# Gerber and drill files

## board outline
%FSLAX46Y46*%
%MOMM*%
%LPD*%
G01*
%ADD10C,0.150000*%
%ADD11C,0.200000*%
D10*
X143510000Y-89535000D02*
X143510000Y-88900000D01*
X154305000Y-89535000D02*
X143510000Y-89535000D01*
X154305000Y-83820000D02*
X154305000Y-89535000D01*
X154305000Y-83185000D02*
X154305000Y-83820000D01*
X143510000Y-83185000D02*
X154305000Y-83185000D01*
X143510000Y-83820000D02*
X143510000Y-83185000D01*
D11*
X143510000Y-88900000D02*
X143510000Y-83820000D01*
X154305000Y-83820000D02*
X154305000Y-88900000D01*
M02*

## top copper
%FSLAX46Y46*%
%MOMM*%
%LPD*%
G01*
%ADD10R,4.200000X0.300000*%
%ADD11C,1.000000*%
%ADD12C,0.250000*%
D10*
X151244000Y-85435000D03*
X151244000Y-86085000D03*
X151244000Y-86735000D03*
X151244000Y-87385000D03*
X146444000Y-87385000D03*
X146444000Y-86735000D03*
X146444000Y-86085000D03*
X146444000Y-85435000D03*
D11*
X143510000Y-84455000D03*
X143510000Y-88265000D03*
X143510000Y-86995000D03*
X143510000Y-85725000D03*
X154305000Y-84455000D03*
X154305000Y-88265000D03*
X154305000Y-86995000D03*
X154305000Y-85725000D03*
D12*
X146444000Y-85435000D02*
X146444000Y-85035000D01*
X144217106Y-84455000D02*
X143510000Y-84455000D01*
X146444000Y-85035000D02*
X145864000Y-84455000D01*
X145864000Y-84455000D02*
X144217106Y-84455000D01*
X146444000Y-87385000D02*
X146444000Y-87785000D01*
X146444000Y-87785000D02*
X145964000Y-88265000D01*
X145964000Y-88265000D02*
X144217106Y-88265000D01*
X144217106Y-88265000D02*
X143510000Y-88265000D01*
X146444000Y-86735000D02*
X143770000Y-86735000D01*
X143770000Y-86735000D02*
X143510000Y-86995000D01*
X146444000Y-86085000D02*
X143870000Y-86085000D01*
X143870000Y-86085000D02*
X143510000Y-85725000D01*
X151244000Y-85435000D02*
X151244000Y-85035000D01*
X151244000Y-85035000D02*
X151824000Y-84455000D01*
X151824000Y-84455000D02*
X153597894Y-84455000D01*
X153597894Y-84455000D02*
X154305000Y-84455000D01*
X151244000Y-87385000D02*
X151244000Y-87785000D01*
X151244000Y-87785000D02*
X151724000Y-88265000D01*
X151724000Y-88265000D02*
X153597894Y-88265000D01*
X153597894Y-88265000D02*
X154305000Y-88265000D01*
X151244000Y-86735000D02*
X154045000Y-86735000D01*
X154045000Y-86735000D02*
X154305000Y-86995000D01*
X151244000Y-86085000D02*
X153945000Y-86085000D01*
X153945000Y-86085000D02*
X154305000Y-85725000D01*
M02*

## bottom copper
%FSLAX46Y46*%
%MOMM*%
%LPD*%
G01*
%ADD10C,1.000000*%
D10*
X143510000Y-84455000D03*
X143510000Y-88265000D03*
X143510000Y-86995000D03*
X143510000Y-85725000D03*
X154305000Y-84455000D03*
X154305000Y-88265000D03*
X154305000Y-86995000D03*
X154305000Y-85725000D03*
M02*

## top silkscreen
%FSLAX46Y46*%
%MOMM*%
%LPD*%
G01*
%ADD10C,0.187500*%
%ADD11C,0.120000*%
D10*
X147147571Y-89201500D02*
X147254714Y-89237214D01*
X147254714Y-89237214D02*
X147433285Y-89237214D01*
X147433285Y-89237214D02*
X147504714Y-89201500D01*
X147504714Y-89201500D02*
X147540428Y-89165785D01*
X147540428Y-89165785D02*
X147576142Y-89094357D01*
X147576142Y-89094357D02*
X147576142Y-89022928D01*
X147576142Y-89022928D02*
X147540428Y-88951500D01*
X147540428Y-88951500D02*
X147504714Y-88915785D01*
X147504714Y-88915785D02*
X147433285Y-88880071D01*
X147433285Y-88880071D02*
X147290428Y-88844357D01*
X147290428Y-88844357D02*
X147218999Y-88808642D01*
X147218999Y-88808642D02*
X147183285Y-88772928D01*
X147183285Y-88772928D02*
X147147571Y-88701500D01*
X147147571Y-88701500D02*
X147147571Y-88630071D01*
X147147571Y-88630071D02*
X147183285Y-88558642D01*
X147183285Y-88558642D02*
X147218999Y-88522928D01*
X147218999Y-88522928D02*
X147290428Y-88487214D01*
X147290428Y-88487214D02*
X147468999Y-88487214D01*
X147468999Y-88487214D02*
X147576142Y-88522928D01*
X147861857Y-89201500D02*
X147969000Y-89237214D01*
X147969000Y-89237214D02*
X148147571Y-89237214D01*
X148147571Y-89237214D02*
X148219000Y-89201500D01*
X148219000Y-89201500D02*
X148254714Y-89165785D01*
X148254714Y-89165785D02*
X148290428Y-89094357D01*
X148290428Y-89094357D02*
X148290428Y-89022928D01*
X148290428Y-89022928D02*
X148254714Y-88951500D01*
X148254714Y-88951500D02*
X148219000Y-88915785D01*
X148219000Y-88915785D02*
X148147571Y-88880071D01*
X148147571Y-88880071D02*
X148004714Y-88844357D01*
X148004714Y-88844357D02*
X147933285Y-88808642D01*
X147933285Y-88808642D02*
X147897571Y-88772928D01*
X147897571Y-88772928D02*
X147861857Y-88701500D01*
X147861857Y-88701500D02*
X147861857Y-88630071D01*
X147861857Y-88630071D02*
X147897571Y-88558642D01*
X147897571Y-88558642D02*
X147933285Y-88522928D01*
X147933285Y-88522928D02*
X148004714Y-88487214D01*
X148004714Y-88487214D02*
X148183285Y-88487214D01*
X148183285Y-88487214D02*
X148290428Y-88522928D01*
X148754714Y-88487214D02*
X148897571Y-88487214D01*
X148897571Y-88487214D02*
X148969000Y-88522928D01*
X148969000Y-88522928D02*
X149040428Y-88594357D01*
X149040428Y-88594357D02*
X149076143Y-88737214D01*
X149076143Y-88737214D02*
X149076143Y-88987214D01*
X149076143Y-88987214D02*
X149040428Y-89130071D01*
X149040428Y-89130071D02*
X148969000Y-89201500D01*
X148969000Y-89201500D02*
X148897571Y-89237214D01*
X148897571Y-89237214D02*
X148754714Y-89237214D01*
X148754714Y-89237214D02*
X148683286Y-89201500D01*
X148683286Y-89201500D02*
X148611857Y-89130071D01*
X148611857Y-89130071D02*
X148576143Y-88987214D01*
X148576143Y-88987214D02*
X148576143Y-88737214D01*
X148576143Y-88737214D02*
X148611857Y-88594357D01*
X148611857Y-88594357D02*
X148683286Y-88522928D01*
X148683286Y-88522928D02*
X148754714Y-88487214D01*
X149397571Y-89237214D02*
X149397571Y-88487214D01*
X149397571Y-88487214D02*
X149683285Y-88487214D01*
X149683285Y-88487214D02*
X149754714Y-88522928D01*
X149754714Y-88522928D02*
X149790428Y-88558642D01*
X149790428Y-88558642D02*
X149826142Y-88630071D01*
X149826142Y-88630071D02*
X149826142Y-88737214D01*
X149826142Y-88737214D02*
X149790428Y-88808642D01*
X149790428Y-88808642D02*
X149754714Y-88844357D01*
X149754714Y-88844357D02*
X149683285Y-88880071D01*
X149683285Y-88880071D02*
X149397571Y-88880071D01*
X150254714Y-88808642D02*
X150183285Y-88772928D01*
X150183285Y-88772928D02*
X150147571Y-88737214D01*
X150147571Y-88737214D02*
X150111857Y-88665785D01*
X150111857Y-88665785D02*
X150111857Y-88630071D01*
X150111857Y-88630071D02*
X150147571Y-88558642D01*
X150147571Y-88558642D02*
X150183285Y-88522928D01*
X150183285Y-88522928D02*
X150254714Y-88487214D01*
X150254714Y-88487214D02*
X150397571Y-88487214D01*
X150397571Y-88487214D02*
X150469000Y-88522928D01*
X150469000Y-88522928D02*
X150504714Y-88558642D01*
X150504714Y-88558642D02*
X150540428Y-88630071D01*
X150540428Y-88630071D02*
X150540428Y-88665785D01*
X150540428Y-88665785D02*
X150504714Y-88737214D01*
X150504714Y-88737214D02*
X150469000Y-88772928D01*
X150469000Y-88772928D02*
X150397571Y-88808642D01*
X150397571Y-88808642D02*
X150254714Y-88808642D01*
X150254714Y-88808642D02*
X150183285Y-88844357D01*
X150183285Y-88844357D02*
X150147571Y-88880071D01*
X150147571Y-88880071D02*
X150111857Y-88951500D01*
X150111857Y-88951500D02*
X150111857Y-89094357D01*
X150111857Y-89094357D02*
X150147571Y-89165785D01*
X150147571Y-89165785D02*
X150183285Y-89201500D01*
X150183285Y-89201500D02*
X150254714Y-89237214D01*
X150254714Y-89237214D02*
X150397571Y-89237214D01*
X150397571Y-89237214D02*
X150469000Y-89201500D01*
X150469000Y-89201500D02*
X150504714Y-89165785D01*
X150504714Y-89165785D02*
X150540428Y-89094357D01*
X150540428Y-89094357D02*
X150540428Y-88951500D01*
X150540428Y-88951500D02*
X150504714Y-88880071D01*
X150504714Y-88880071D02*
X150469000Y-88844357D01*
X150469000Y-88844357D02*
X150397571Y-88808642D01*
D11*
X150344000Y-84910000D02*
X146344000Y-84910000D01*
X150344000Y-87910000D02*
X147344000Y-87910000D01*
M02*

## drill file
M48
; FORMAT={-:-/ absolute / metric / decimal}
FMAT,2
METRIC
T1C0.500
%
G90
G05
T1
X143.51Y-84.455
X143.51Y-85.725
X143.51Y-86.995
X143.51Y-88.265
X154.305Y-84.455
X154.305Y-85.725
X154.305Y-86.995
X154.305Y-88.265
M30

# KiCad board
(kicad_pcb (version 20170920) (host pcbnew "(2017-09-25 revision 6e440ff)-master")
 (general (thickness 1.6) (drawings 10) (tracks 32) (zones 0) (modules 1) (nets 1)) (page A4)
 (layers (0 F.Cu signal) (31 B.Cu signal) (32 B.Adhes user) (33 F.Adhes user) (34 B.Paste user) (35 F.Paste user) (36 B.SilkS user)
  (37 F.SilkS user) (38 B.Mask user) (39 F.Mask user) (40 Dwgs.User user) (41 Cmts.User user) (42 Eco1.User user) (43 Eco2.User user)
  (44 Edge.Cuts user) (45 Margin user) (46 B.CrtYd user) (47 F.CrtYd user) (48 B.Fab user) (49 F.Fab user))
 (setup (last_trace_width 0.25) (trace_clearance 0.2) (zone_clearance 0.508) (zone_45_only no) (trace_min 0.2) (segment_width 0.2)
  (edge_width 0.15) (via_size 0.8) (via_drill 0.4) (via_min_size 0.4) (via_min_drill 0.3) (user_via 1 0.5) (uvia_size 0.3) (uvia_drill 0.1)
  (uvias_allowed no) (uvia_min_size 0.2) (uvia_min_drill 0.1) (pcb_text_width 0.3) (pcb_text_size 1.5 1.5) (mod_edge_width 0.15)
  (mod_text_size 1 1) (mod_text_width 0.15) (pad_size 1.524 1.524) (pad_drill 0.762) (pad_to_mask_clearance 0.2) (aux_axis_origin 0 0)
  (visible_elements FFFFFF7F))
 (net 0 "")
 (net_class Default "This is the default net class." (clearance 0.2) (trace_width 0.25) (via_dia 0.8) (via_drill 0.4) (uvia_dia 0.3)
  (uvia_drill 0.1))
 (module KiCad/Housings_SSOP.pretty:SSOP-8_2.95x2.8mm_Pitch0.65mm (layer F.Cu) (at 148.844 86.41)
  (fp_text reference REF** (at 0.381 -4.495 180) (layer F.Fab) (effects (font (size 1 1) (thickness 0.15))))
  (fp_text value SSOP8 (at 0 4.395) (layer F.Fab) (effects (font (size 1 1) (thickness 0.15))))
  (fp_line (start 1.5 -1.5) (end -2.5 -1.5) (layer F.SilkS) (width 0.12))
  (fp_line (start 1.5 1.5) (end -1.5 1.5) (layer F.SilkS) (width 0.12))
  (pad 8 smd rect (at 2.4 -0.975 270) (size 0.3 4.2) (layers F.Cu F.Paste F.Mask))
  (pad 7 smd rect (at 2.4 -0.325 270) (size 0.3 4.2) (layers F.Cu F.Paste F.Mask))
  (pad 6 smd rect (at 2.4 0.325 270) (size 0.3 4.2) (layers F.Cu F.Paste F.Mask))
  (pad 5 smd rect (at 2.4 0.975 270) (size 0.3 4.2) (layers F.Cu F.Paste F.Mask))
  (pad 4 smd rect (at -2.4 0.975 270) (size 0.3 4.2) (layers F.Cu F.Paste F.Mask))
  (pad 3 smd rect (at -2.4 0.325 270) (size 0.3 4.2) (layers F.Cu F.Paste F.Mask))
  (pad 2 smd rect (at -2.4 -0.325 270) (size 0.3 4.2) (layers F.Cu F.Paste F.Mask))
  (pad 1 smd rect (at -2.4 -0.975 270) (size 0.3 4.2) (layers F.Cu F.Paste F.Mask)))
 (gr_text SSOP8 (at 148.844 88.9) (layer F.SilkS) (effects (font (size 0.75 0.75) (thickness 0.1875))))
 (gr_line (start 143.51 89.535) (end 143.51 88.9) (layer Edge.Cuts) (width 0.15))
 (gr_line (start 154.305 89.535) (end 143.51 89.535) (layer Edge.Cuts) (width 0.15))
 (gr_line (start 154.305 83.82) (end 154.305 89.535) (layer Edge.Cuts) (width 0.15))
 (gr_line (start 154.305 83.185) (end 154.305 83.82) (layer Edge.Cuts) (width 0.15))
 (gr_line (start 143.51 83.185) (end 154.305 83.185) (layer Edge.Cuts) (width 0.15))
 (gr_line (start 143.51 83.82) (end 143.51 83.185) (layer Edge.Cuts) (width 0.15))
 (gr_line (start 143.51 88.9) (end 143.51 83.82) (layer Edge.Cuts) (width 0.2))
 (gr_line (start 154.305 83.82) (end 154.305 88.9) (layer Edge.Cuts) (width 0.2))
 (segment (start 146.444 85.435) (end 146.444 85.035) (width 0.25) (layer F.Cu) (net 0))
 (segment (start 144.217106 84.455) (end 143.51 84.455) (width 0.25) (layer F.Cu) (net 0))
 (segment (start 146.444 85.035) (end 145.864 84.455) (width 0.25) (layer F.Cu) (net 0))
 (segment (start 145.864 84.455) (end 144.217106 84.455) (width 0.25) (layer F.Cu) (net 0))
 (segment (start 146.444 87.385) (end 146.444 87.785) (width 0.25) (layer F.Cu) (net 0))
 (segment (start 146.444 87.785) (end 145.964 88.265) (width 0.25) (layer F.Cu) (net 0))
 (segment (start 145.964 88.265) (end 144.217106 88.265) (width 0.25) (layer F.Cu) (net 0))
 (segment (start 144.217106 88.265) (end 143.51 88.265) (width 0.25) (layer F.Cu) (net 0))
 (segment (start 146.444 86.735) (end 143.77 86.735) (width 0.25) (layer F.Cu) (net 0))
 (segment (start 143.77 86.735) (end 143.51 86.995) (width 0.25) (layer F.Cu) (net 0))
 (segment (start 146.444 86.085) (end 143.87 86.085) (width 0.25) (layer F.Cu) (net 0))
 (segment (start 143.87 86.085) (end 143.51 85.725) (width 0.25) (layer F.Cu) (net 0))
 (segment (start 151.244 85.435) (end 151.244 85.035) (width 0.25) (layer F.Cu) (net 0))
 (segment (start 151.244 85.035) (end 151.824 84.455) (width 0.25) (layer F.Cu) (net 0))
 (segment (start 151.824 84.455) (end 153.597894 84.455) (width 0.25) (layer F.Cu) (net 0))
 (segment (start 153.597894 84.455) (end 154.305 84.455) (width 0.25) (layer F.Cu) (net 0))
 (segment (start 151.244 87.385) (end 151.244 87.785) (width 0.25) (layer F.Cu) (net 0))
 (segment (start 151.244 87.785) (end 151.724 88.265) (width 0.25) (layer F.Cu) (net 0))
 (segment (start 151.724 88.265) (end 153.597894 88.265) (width 0.25) (layer F.Cu) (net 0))
 (segment (start 153.597894 88.265) (end 154.305 88.265) (width 0.25) (layer F.Cu) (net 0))
 (segment (start 151.244 86.735) (end 154.045 86.735) (width 0.25) (layer F.Cu) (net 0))
 (segment (start 154.045 86.735) (end 154.305 86.995) (width 0.25) (layer F.Cu) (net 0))
 (segment (start 151.244 86.085) (end 153.945 86.085) (width 0.25) (layer F.Cu) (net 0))
 (segment (start 153.945 86.085) (end 154.305 85.725) (width 0.25) (layer F.Cu) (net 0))
 (via (at 143.51 84.455) (size 1) (drill 0.5) (layers F.Cu B.Cu) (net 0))
 (via (at 143.51 88.265) (size 1) (drill 0.5) (layers F.Cu B.Cu) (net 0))
 (via (at 143.51 86.995) (size 1) (drill 0.5) (layers F.Cu B.Cu) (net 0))
 (via (at 143.51 85.725) (size 1) (drill 0.5) (layers F.Cu B.Cu) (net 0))
 (via (at 154.305 84.455) (size 1) (drill 0.5) (layers F.Cu B.Cu) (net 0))
 (via (at 154.305 88.265) (size 1) (drill 0.5) (layers F.Cu B.Cu) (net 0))
 (via (at 154.305 86.995) (size 1) (drill 0.5) (layers F.Cu B.Cu) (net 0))
 (via (at 154.305 85.725) (size 1) (drill 0.5) (layers F.Cu B.Cu) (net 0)))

